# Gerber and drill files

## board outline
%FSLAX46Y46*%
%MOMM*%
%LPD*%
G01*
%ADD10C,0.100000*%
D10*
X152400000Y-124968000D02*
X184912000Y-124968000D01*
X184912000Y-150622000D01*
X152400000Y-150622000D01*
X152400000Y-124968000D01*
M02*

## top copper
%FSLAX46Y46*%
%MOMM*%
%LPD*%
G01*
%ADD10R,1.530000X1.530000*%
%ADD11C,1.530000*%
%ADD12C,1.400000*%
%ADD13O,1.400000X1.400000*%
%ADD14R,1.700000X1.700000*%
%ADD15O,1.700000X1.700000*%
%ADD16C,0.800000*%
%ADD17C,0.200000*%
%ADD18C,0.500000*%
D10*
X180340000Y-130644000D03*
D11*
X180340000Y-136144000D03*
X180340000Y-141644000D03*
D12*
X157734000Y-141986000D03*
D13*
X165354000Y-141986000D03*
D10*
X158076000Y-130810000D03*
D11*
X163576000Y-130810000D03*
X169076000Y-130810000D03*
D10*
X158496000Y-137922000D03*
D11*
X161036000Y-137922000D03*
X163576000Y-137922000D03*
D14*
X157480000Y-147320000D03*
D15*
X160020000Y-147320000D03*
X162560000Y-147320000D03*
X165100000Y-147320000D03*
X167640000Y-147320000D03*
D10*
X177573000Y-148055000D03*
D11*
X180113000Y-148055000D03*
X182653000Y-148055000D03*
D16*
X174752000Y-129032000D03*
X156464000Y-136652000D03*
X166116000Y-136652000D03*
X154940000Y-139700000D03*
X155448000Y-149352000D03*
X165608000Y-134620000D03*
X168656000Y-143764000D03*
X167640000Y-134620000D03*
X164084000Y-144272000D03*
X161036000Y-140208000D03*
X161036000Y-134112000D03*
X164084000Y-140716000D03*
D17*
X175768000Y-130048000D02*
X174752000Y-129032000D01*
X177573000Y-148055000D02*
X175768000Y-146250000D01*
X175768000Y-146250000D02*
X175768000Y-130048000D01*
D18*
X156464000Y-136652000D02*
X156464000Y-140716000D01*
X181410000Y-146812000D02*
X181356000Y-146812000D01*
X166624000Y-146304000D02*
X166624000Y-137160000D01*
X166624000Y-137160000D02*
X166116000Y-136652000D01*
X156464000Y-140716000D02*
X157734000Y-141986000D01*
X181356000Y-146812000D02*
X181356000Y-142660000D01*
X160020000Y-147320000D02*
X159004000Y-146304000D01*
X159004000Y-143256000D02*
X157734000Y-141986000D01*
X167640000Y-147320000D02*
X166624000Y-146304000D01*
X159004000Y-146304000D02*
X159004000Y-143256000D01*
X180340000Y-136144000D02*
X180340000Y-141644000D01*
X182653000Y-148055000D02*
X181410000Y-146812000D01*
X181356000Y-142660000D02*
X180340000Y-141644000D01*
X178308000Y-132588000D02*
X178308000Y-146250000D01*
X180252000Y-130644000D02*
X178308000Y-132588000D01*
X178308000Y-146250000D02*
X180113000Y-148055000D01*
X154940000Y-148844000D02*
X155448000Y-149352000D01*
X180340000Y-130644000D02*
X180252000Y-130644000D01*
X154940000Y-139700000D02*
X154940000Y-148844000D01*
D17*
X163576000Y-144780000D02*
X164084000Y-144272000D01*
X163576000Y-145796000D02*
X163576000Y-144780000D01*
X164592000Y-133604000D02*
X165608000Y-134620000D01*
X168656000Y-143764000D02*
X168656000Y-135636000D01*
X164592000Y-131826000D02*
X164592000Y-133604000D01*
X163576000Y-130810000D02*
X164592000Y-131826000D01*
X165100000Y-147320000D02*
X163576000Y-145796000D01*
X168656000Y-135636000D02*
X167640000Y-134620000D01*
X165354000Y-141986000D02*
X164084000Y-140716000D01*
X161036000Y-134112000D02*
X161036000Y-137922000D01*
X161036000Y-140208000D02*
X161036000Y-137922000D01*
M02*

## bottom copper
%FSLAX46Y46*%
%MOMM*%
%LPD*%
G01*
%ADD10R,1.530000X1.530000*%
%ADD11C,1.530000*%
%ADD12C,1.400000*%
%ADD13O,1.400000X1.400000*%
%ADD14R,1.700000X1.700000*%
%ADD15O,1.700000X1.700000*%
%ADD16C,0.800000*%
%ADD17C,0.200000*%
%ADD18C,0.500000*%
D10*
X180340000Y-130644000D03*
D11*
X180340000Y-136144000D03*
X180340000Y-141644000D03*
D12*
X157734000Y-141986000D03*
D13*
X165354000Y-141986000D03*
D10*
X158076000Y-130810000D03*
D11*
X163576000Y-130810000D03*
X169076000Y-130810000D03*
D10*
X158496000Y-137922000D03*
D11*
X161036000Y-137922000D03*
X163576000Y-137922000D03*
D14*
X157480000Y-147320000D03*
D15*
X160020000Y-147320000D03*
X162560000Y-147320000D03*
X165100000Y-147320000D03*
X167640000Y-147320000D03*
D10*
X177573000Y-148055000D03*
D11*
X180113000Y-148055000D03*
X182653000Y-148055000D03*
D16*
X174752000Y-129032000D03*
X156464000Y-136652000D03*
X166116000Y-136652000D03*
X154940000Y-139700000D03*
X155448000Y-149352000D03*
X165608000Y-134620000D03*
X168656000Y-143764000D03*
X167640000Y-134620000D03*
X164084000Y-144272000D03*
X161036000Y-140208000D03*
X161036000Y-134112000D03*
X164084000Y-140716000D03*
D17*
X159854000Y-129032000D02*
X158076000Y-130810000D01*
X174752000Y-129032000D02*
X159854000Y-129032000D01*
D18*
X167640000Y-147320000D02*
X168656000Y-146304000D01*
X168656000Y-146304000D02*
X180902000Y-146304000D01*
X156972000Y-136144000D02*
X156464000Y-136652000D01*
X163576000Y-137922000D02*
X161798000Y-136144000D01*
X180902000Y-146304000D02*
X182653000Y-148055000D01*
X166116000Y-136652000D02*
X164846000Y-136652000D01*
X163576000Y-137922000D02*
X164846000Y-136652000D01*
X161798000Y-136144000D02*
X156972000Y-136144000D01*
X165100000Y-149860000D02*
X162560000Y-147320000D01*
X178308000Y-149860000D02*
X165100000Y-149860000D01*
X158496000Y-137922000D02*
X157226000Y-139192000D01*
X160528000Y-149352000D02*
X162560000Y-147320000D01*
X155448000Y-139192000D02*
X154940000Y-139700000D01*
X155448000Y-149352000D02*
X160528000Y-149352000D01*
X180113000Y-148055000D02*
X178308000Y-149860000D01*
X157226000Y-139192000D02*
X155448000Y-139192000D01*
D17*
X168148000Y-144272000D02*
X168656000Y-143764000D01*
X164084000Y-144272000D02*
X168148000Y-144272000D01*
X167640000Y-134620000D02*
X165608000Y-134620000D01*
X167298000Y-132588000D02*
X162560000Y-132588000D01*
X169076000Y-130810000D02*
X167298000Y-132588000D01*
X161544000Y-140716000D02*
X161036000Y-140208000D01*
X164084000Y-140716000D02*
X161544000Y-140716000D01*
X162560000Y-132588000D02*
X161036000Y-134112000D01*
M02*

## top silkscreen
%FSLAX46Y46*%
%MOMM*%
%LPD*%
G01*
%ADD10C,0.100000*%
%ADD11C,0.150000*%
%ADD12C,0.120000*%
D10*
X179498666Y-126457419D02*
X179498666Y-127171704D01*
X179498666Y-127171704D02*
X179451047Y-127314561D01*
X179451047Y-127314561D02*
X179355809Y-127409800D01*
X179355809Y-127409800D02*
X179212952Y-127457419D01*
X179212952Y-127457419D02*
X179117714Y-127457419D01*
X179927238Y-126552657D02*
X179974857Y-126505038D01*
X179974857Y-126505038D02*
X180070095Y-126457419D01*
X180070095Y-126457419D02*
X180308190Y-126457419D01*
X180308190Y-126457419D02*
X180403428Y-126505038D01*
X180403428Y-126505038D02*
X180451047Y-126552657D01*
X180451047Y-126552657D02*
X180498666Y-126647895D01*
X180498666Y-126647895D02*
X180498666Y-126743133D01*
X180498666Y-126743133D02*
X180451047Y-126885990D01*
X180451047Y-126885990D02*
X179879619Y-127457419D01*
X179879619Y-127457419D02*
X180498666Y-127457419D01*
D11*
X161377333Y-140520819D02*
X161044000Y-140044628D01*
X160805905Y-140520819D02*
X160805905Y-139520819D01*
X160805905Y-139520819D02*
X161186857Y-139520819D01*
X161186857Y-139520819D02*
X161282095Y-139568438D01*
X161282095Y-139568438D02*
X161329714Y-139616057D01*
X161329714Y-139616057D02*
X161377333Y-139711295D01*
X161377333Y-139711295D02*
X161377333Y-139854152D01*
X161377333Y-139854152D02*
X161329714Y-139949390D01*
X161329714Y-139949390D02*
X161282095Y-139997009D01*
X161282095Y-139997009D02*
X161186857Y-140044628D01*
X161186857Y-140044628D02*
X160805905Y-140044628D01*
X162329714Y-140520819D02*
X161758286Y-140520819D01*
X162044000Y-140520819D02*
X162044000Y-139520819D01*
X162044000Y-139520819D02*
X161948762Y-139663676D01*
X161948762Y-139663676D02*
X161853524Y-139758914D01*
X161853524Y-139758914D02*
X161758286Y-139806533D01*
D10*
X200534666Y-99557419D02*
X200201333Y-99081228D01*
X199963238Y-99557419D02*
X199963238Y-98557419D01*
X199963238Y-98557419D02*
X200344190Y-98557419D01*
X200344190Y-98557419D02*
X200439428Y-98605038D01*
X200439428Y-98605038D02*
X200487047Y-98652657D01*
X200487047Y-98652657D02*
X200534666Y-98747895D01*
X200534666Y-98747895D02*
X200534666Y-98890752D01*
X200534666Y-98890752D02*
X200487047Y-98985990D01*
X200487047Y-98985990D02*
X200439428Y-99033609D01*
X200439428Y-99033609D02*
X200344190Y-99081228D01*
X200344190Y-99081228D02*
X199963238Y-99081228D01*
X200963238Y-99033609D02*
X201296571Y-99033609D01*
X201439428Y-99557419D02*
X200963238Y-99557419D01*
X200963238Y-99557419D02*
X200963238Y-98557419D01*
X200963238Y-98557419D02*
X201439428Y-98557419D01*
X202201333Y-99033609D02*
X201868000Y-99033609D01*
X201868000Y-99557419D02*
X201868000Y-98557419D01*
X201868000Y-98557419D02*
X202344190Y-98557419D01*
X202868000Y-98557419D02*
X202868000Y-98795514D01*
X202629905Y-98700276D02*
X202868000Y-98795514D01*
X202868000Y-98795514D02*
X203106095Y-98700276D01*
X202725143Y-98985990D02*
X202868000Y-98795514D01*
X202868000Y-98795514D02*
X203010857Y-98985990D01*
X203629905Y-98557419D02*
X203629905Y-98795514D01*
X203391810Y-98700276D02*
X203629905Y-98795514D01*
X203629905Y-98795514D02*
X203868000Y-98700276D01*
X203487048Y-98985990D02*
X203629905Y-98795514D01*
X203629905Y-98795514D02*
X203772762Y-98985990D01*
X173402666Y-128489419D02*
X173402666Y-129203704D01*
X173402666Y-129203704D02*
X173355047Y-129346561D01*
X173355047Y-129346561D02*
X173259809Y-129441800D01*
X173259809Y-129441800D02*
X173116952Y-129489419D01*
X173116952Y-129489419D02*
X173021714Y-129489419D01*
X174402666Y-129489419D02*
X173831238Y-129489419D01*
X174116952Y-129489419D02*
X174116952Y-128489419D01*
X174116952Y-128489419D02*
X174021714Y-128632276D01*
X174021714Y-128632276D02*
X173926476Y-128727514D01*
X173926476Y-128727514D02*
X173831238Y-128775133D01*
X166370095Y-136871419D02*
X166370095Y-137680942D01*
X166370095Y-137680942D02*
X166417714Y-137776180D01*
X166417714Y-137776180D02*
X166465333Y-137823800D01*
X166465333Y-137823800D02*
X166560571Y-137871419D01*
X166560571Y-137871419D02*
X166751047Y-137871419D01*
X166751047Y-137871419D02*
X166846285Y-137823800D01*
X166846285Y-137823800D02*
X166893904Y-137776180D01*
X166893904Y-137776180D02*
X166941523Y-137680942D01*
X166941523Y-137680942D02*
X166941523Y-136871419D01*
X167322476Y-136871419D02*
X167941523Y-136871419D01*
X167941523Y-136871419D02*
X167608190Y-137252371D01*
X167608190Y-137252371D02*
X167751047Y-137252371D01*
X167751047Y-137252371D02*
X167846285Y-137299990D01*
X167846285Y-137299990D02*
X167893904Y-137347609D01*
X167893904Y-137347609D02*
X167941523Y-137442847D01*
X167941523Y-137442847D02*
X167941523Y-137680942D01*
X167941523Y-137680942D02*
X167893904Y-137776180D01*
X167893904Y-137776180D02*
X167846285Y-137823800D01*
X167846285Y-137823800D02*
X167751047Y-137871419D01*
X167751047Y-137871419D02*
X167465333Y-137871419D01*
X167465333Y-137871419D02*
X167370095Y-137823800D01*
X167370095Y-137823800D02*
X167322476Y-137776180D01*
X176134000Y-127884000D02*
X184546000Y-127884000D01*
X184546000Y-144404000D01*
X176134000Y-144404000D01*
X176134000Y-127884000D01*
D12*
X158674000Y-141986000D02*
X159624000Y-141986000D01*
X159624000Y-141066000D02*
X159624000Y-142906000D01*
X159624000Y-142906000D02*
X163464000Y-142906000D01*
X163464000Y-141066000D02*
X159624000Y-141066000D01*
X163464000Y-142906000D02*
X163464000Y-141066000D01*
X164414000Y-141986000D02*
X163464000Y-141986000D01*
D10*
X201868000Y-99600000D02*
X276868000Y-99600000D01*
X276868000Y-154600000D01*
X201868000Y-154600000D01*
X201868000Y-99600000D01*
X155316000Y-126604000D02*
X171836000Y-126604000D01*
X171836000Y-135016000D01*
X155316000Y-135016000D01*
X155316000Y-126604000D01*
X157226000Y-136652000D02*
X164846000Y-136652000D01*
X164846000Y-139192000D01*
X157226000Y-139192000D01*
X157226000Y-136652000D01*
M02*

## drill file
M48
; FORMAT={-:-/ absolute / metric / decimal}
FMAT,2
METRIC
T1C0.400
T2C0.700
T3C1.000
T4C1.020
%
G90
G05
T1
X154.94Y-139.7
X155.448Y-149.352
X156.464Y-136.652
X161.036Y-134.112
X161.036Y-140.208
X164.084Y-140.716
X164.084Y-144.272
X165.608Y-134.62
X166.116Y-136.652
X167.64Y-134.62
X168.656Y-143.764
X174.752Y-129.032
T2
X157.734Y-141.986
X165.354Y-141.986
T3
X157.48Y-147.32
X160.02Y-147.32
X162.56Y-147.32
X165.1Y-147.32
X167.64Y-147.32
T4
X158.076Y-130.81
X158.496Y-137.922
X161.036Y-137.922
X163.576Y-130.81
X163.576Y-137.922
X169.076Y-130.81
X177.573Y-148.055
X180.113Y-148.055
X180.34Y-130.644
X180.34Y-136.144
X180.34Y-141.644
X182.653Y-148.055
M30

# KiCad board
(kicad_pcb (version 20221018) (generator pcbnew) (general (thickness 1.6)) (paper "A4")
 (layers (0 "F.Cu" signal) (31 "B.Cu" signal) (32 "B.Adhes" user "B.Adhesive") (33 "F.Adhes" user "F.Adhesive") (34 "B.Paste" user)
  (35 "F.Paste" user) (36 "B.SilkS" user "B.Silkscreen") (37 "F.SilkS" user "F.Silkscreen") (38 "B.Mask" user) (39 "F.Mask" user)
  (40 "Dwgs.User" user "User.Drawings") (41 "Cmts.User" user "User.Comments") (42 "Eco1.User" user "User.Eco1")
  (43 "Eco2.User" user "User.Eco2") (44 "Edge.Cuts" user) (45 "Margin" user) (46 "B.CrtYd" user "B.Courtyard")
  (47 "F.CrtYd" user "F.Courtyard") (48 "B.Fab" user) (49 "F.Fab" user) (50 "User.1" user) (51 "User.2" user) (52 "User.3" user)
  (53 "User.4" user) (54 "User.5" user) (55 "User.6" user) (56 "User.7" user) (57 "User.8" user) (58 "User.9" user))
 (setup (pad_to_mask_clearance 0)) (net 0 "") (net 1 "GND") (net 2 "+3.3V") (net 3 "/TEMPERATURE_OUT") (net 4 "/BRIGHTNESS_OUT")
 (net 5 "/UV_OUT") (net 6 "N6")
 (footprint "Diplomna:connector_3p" (layer "F.Cu") (at 180.34 136.144 -90)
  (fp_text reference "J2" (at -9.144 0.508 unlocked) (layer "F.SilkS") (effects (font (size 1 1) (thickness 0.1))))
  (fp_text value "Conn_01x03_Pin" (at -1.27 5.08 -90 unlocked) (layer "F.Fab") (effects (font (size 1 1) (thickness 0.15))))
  (fp_rect (start -8.26 -4.206) (end 8.26 4.206) (stroke (width 0.1) (type default)) (fill none) (layer "F.SilkS"))
  (pad "1" thru_hole rect (at -5.5 0 270) (size 1.53 1.53) (drill 1.02) (layers "*.Cu" "*.Mask") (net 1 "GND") (solder_mask_margin 0.102))
  (pad "2" thru_hole circle (at 0 0 270) (size 1.53 1.53) (drill 1.02) (layers "*.Cu" "*.Mask") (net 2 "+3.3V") (solder_mask_margin 0.102))
  (pad "3" thru_hole circle (at 5.5 0 270) (size 1.53 1.53) (drill 1.02) (layers "*.Cu" "*.Mask") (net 2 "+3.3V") (solder_mask_margin 0.102)))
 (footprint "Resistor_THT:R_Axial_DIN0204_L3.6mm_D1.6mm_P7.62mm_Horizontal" (layer "F.Cu") (at 157.734 141.986)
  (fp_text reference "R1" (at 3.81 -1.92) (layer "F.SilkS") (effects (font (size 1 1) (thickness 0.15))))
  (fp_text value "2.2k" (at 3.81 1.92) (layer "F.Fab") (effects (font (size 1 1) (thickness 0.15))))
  (fp_line (start 0.94 0) (end 1.89 0) (stroke (width 0.12) (type solid)) (layer "F.SilkS"))
  (fp_line (start 1.89 -0.92) (end 1.89 0.92) (stroke (width 0.12) (type solid)) (layer "F.SilkS"))
  (fp_line (start 1.89 0.92) (end 5.73 0.92) (stroke (width 0.12) (type solid)) (layer "F.SilkS"))
  (fp_line (start 5.73 -0.92) (end 1.89 -0.92) (stroke (width 0.12) (type solid)) (layer "F.SilkS"))
  (fp_line (start 5.73 0.92) (end 5.73 -0.92) (stroke (width 0.12) (type solid)) (layer "F.SilkS"))
  (fp_line (start 6.68 0) (end 5.73 0) (stroke (width 0.12) (type solid)) (layer "F.SilkS"))
  (pad "1" thru_hole circle (at 0 0) (size 1.4 1.4) (drill 0.7) (layers "*.Cu" "*.Mask") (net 2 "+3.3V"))
  (pad "2" thru_hole oval (at 7.62 0) (size 1.4 1.4) (drill 0.7) (layers "*.Cu" "*.Mask") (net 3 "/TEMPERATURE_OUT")))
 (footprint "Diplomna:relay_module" (layer "F.Cu") (at 201.868 99.6)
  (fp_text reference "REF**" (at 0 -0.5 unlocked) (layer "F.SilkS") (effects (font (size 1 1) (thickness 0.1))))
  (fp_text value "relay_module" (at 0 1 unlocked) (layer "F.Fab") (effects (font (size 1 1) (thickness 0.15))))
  (fp_rect (start 0 0) (end 75 55) (stroke (width 0.1) (type default)) (fill none) (layer "F.SilkS")))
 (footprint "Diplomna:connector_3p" (layer "F.Cu") (at 163.576 130.81)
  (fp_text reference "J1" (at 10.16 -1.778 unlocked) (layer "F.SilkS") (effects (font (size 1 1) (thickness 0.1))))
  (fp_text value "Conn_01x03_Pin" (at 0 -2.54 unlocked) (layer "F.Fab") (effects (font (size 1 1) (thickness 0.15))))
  (fp_rect (start -8.26 -4.206) (end 8.26 4.206) (stroke (width 0.1) (type default)) (fill none) (layer "F.SilkS"))
  (pad "1" thru_hole rect (at -5.5 0) (size 1.53 1.53) (drill 1.02) (layers "*.Cu" "*.Mask") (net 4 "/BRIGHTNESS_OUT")
   (solder_mask_margin 0.102))
  (pad "2" thru_hole circle (at 0 0) (size 1.53 1.53) (drill 1.02) (layers "*.Cu" "*.Mask") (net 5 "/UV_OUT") (solder_mask_margin 0.102))
  (pad "3" thru_hole circle (at 5.5 0) (size 1.53 1.53) (drill 1.02) (layers "*.Cu" "*.Mask") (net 3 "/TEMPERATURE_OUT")
   (solder_mask_margin 0.102)))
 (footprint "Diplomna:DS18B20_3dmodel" (layer "F.Cu") (at 166.116 140.462)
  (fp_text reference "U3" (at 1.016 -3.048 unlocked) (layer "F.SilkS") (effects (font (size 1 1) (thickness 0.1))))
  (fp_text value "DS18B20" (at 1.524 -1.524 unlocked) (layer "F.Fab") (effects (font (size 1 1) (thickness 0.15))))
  (fp_rect (start -8.89 -3.81) (end -1.27 -1.27) (stroke (width 0.1) (type default)) (fill none) (layer "F.SilkS"))
  (pad "1" thru_hole rect (at -7.62 -2.54) (size 1.53 1.53) (drill 1.02) (layers "*.Cu" "*.Mask") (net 1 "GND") (solder_mask_margin 0.102))
  (pad "2" thru_hole circle (at -5.08 -2.54) (size 1.53 1.53) (drill 1.02) (layers "*.Cu" "*.Mask") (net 3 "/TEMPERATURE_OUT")
   (solder_mask_margin 0.102))
  (pad "3" thru_hole circle (at -2.54 -2.54) (size 1.53 1.53) (drill 1.02) (layers "*.Cu" "*.Mask") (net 2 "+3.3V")
   (solder_mask_margin 0.102)))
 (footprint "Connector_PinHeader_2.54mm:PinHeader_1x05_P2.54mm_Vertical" (layer "B.Cu") (at 157.48 147.32 -90)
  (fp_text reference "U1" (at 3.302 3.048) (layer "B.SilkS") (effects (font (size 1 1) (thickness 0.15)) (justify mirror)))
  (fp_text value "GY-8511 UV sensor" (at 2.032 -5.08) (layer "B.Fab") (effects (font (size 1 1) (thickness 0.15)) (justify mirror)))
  (pad "1" thru_hole rect (at 0 0 270) (size 1.7 1.7) (drill 1) (layers "*.Cu" "*.Mask") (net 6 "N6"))
  (pad "2" thru_hole oval (at 0 -2.54 270) (size 1.7 1.7) (drill 1) (layers "*.Cu" "*.Mask") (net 2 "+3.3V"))
  (pad "3" thru_hole oval (at 0 -5.08 270) (size 1.7 1.7) (drill 1) (layers "*.Cu" "*.Mask") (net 1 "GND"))
  (pad "4" thru_hole oval (at 0 -7.62 270) (size 1.7 1.7) (drill 1) (layers "*.Cu" "*.Mask") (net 5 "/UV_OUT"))
  (pad "5" thru_hole oval (at 0 -10.16 270) (size 1.7 1.7) (drill 1) (layers "*.Cu" "*.Mask") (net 2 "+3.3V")))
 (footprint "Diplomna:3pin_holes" (layer "B.Cu") (at 185.193 145.515)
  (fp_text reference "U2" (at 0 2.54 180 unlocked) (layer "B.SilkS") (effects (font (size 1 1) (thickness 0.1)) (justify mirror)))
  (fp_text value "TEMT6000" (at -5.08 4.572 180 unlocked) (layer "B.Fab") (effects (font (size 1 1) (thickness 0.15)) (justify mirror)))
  (pad "1" thru_hole rect (at -7.62 2.54) (size 1.53 1.53) (drill 1.02) (layers "*.Cu" "*.Mask") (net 4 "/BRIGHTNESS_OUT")
   (solder_mask_margin 0.102))
  (pad "2" thru_hole circle (at -5.08 2.54) (size 1.53 1.53) (drill 1.02) (layers "*.Cu" "*.Mask") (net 1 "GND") (solder_mask_margin 0.102))
  (pad "3" thru_hole circle (at -2.54 2.54) (size 1.53 1.53) (drill 1.02) (layers "*.Cu" "*.Mask") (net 2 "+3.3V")
   (solder_mask_margin 0.102)))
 (gr_rect (start 152.4 124.968) (end 184.912 150.622) (stroke (width 0.1) (type default)) (fill none) (layer "Edge.Cuts"))
 (segment (start 175.768 130.048) (end 174.752 129.032) (width 0.2) (layer "F.Cu") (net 4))
 (segment (start 177.573 148.055) (end 175.768 146.25) (width 0.2) (layer "F.Cu") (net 4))
 (segment (start 175.768 146.25) (end 175.768 130.048) (width 0.2) (layer "F.Cu") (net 4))
 (via (at 174.752 129.032) (size 0.8) (drill 0.4) (layers "F.Cu" "B.Cu") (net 4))
 (segment (start 159.854 129.032) (end 158.076 130.81) (width 0.2) (layer "B.Cu") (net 4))
 (segment (start 174.752 129.032) (end 159.854 129.032) (width 0.2) (layer "B.Cu") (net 4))
 (segment (start 156.464 136.652) (end 156.464 140.716) (width 0.5) (layer "F.Cu") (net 2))
 (segment (start 181.41 146.812) (end 181.356 146.812) (width 0.5) (layer "F.Cu") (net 2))
 (segment (start 166.624 146.304) (end 166.624 137.16) (width 0.5) (layer "F.Cu") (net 2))
 (segment (start 166.624 137.16) (end 166.116 136.652) (width 0.5) (layer "F.Cu") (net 2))
 (segment (start 156.464 140.716) (end 157.734 141.986) (width 0.5) (layer "F.Cu") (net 2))
 (segment (start 181.356 146.812) (end 181.356 142.66) (width 0.5) (layer "F.Cu") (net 2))
 (segment (start 160.02 147.32) (end 159.004 146.304) (width 0.5) (layer "F.Cu") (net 2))
 (segment (start 159.004 143.256) (end 157.734 141.986) (width 0.5) (layer "F.Cu") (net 2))
 (segment (start 167.64 147.32) (end 166.624 146.304) (width 0.5) (layer "F.Cu") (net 2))
 (segment (start 159.004 146.304) (end 159.004 143.256) (width 0.5) (layer "F.Cu") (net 2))
 (segment (start 180.34 136.144) (end 180.34 141.644) (width 0.5) (layer "F.Cu") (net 2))
 (segment (start 182.653 148.055) (end 181.41 146.812) (width 0.5) (layer "F.Cu") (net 2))
 (segment (start 181.356 142.66) (end 180.34 141.644) (width 0.5) (layer "F.Cu") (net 2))
 (via (at 156.464 136.652) (size 0.8) (drill 0.4) (layers "F.Cu" "B.Cu") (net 2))
 (via (at 166.116 136.652) (size 0.8) (drill 0.4) (layers "F.Cu" "B.Cu") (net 2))
 (segment (start 167.64 147.32) (end 168.656 146.304) (width 0.5) (layer "B.Cu") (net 2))
 (segment (start 168.656 146.304) (end 180.902 146.304) (width 0.5) (layer "B.Cu") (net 2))
 (segment (start 156.972 136.144) (end 156.464 136.652) (width 0.5) (layer "B.Cu") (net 2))
 (segment (start 163.576 137.922) (end 161.798 136.144) (width 0.5) (layer "B.Cu") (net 2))
 (segment (start 180.902 146.304) (end 182.653 148.055) (width 0.5) (layer "B.Cu") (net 2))
 (segment (start 166.116 136.652) (end 164.846 136.652) (width 0.5) (layer "B.Cu") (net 2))
 (segment (start 163.576 137.922) (end 164.846 136.652) (width 0.5) (layer "B.Cu") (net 2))
 (segment (start 161.798 136.144) (end 156.972 136.144) (width 0.5) (layer "B.Cu") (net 2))
 (segment (start 178.308 132.588) (end 178.308 146.25) (width 0.5) (layer "F.Cu") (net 1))
 (segment (start 180.252 130.644) (end 178.308 132.588) (width 0.5) (layer "F.Cu") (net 1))
 (segment (start 178.308 146.25) (end 180.113 148.055) (width 0.5) (layer "F.Cu") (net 1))
 (segment (start 154.94 148.844) (end 155.448 149.352) (width 0.5) (layer "F.Cu") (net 1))
 (segment (start 180.34 130.644) (end 180.252 130.644) (width 0.5) (layer "F.Cu") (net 1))
 (segment (start 154.94 139.7) (end 154.94 148.844) (width 0.5) (layer "F.Cu") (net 1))
 (via (at 154.94 139.7) (size 0.8) (drill 0.4) (layers "F.Cu" "B.Cu") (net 1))
 (via (at 155.448 149.352) (size 0.8) (drill 0.4) (layers "F.Cu" "B.Cu") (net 1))
 (segment (start 165.1 149.86) (end 162.56 147.32) (width 0.5) (layer "B.Cu") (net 1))
 (segment (start 178.308 149.86) (end 165.1 149.86) (width 0.5) (layer "B.Cu") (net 1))
 (segment (start 158.496 137.922) (end 157.226 139.192) (width 0.5) (layer "B.Cu") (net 1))
 (segment (start 160.528 149.352) (end 162.56 147.32) (width 0.5) (layer "B.Cu") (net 1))
 (segment (start 155.448 139.192) (end 154.94 139.7) (width 0.5) (layer "B.Cu") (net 1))
 (segment (start 155.448 149.352) (end 160.528 149.352) (width 0.5) (layer "B.Cu") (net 1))
 (segment (start 180.113 148.055) (end 178.308 149.86) (width 0.5) (layer "B.Cu") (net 1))
 (segment (start 157.226 139.192) (end 155.448 139.192) (width 0.5) (layer "B.Cu") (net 1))
 (segment (start 163.576 144.78) (end 164.084 144.272) (width 0.2) (layer "F.Cu") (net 5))
 (segment (start 163.576 145.796) (end 163.576 144.78) (width 0.2) (layer "F.Cu") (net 5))
 (segment (start 164.592 133.604) (end 165.608 134.62) (width 0.2) (layer "F.Cu") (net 5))
 (segment (start 168.656 143.764) (end 168.656 135.636) (width 0.2) (layer "F.Cu") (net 5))
 (segment (start 164.592 131.826) (end 164.592 133.604) (width 0.2) (layer "F.Cu") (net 5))
 (segment (start 163.576 130.81) (end 164.592 131.826) (width 0.2) (layer "F.Cu") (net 5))
 (segment (start 165.1 147.32) (end 163.576 145.796) (width 0.2) (layer "F.Cu") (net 5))
 (segment (start 168.656 135.636) (end 167.64 134.62) (width 0.2) (layer "F.Cu") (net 5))
 (via (at 165.608 134.62) (size 0.8) (drill 0.4) (layers "F.Cu" "B.Cu") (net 5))
 (via (at 168.656 143.764) (size 0.8) (drill 0.4) (layers "F.Cu" "B.Cu") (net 5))
 (via (at 167.64 134.62) (size 0.8) (drill 0.4) (layers "F.Cu" "B.Cu") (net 5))
 (via (at 164.084 144.272) (size 0.8) (drill 0.4) (layers "F.Cu" "B.Cu") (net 5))
 (segment (start 168.148 144.272) (end 168.656 143.764) (width 0.2) (layer "B.Cu") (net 5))
 (segment (start 164.084 144.272) (end 168.148 144.272) (width 0.2) (layer "B.Cu") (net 5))
 (segment (start 167.64 134.62) (end 165.608 134.62) (width 0.2) (layer "B.Cu") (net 5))
 (segment (start 165.354 141.986) (end 164.084 140.716) (width 0.2) (layer "F.Cu") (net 3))
 (segment (start 161.036 134.112) (end 161.036 137.922) (width 0.2) (layer "F.Cu") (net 3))
 (segment (start 161.036 140.208) (end 161.036 137.922) (width 0.2) (layer "F.Cu") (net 3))
 (via (at 161.036 140.208) (size 0.8) (drill 0.4) (layers "F.Cu" "B.Cu") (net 3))
 (via (at 161.036 134.112) (size 0.8) (drill 0.4) (layers "F.Cu" "B.Cu") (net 3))
 (via (at 164.084 140.716) (size 0.8) (drill 0.4) (layers "F.Cu" "B.Cu") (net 3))
 (segment (start 167.298 132.588) (end 162.56 132.588) (width 0.2) (layer "B.Cu") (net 3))
 (segment (start 169.076 130.81) (end 167.298 132.588) (width 0.2) (layer "B.Cu") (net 3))
 (segment (start 161.544 140.716) (end 161.036 140.208) (width 0.2) (layer "B.Cu") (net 3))
 (segment (start 164.084 140.716) (end 161.544 140.716) (width 0.2) (layer "B.Cu") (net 3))
 (segment (start 162.56 132.588) (end 161.036 134.112) (width 0.2) (layer "B.Cu") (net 3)))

